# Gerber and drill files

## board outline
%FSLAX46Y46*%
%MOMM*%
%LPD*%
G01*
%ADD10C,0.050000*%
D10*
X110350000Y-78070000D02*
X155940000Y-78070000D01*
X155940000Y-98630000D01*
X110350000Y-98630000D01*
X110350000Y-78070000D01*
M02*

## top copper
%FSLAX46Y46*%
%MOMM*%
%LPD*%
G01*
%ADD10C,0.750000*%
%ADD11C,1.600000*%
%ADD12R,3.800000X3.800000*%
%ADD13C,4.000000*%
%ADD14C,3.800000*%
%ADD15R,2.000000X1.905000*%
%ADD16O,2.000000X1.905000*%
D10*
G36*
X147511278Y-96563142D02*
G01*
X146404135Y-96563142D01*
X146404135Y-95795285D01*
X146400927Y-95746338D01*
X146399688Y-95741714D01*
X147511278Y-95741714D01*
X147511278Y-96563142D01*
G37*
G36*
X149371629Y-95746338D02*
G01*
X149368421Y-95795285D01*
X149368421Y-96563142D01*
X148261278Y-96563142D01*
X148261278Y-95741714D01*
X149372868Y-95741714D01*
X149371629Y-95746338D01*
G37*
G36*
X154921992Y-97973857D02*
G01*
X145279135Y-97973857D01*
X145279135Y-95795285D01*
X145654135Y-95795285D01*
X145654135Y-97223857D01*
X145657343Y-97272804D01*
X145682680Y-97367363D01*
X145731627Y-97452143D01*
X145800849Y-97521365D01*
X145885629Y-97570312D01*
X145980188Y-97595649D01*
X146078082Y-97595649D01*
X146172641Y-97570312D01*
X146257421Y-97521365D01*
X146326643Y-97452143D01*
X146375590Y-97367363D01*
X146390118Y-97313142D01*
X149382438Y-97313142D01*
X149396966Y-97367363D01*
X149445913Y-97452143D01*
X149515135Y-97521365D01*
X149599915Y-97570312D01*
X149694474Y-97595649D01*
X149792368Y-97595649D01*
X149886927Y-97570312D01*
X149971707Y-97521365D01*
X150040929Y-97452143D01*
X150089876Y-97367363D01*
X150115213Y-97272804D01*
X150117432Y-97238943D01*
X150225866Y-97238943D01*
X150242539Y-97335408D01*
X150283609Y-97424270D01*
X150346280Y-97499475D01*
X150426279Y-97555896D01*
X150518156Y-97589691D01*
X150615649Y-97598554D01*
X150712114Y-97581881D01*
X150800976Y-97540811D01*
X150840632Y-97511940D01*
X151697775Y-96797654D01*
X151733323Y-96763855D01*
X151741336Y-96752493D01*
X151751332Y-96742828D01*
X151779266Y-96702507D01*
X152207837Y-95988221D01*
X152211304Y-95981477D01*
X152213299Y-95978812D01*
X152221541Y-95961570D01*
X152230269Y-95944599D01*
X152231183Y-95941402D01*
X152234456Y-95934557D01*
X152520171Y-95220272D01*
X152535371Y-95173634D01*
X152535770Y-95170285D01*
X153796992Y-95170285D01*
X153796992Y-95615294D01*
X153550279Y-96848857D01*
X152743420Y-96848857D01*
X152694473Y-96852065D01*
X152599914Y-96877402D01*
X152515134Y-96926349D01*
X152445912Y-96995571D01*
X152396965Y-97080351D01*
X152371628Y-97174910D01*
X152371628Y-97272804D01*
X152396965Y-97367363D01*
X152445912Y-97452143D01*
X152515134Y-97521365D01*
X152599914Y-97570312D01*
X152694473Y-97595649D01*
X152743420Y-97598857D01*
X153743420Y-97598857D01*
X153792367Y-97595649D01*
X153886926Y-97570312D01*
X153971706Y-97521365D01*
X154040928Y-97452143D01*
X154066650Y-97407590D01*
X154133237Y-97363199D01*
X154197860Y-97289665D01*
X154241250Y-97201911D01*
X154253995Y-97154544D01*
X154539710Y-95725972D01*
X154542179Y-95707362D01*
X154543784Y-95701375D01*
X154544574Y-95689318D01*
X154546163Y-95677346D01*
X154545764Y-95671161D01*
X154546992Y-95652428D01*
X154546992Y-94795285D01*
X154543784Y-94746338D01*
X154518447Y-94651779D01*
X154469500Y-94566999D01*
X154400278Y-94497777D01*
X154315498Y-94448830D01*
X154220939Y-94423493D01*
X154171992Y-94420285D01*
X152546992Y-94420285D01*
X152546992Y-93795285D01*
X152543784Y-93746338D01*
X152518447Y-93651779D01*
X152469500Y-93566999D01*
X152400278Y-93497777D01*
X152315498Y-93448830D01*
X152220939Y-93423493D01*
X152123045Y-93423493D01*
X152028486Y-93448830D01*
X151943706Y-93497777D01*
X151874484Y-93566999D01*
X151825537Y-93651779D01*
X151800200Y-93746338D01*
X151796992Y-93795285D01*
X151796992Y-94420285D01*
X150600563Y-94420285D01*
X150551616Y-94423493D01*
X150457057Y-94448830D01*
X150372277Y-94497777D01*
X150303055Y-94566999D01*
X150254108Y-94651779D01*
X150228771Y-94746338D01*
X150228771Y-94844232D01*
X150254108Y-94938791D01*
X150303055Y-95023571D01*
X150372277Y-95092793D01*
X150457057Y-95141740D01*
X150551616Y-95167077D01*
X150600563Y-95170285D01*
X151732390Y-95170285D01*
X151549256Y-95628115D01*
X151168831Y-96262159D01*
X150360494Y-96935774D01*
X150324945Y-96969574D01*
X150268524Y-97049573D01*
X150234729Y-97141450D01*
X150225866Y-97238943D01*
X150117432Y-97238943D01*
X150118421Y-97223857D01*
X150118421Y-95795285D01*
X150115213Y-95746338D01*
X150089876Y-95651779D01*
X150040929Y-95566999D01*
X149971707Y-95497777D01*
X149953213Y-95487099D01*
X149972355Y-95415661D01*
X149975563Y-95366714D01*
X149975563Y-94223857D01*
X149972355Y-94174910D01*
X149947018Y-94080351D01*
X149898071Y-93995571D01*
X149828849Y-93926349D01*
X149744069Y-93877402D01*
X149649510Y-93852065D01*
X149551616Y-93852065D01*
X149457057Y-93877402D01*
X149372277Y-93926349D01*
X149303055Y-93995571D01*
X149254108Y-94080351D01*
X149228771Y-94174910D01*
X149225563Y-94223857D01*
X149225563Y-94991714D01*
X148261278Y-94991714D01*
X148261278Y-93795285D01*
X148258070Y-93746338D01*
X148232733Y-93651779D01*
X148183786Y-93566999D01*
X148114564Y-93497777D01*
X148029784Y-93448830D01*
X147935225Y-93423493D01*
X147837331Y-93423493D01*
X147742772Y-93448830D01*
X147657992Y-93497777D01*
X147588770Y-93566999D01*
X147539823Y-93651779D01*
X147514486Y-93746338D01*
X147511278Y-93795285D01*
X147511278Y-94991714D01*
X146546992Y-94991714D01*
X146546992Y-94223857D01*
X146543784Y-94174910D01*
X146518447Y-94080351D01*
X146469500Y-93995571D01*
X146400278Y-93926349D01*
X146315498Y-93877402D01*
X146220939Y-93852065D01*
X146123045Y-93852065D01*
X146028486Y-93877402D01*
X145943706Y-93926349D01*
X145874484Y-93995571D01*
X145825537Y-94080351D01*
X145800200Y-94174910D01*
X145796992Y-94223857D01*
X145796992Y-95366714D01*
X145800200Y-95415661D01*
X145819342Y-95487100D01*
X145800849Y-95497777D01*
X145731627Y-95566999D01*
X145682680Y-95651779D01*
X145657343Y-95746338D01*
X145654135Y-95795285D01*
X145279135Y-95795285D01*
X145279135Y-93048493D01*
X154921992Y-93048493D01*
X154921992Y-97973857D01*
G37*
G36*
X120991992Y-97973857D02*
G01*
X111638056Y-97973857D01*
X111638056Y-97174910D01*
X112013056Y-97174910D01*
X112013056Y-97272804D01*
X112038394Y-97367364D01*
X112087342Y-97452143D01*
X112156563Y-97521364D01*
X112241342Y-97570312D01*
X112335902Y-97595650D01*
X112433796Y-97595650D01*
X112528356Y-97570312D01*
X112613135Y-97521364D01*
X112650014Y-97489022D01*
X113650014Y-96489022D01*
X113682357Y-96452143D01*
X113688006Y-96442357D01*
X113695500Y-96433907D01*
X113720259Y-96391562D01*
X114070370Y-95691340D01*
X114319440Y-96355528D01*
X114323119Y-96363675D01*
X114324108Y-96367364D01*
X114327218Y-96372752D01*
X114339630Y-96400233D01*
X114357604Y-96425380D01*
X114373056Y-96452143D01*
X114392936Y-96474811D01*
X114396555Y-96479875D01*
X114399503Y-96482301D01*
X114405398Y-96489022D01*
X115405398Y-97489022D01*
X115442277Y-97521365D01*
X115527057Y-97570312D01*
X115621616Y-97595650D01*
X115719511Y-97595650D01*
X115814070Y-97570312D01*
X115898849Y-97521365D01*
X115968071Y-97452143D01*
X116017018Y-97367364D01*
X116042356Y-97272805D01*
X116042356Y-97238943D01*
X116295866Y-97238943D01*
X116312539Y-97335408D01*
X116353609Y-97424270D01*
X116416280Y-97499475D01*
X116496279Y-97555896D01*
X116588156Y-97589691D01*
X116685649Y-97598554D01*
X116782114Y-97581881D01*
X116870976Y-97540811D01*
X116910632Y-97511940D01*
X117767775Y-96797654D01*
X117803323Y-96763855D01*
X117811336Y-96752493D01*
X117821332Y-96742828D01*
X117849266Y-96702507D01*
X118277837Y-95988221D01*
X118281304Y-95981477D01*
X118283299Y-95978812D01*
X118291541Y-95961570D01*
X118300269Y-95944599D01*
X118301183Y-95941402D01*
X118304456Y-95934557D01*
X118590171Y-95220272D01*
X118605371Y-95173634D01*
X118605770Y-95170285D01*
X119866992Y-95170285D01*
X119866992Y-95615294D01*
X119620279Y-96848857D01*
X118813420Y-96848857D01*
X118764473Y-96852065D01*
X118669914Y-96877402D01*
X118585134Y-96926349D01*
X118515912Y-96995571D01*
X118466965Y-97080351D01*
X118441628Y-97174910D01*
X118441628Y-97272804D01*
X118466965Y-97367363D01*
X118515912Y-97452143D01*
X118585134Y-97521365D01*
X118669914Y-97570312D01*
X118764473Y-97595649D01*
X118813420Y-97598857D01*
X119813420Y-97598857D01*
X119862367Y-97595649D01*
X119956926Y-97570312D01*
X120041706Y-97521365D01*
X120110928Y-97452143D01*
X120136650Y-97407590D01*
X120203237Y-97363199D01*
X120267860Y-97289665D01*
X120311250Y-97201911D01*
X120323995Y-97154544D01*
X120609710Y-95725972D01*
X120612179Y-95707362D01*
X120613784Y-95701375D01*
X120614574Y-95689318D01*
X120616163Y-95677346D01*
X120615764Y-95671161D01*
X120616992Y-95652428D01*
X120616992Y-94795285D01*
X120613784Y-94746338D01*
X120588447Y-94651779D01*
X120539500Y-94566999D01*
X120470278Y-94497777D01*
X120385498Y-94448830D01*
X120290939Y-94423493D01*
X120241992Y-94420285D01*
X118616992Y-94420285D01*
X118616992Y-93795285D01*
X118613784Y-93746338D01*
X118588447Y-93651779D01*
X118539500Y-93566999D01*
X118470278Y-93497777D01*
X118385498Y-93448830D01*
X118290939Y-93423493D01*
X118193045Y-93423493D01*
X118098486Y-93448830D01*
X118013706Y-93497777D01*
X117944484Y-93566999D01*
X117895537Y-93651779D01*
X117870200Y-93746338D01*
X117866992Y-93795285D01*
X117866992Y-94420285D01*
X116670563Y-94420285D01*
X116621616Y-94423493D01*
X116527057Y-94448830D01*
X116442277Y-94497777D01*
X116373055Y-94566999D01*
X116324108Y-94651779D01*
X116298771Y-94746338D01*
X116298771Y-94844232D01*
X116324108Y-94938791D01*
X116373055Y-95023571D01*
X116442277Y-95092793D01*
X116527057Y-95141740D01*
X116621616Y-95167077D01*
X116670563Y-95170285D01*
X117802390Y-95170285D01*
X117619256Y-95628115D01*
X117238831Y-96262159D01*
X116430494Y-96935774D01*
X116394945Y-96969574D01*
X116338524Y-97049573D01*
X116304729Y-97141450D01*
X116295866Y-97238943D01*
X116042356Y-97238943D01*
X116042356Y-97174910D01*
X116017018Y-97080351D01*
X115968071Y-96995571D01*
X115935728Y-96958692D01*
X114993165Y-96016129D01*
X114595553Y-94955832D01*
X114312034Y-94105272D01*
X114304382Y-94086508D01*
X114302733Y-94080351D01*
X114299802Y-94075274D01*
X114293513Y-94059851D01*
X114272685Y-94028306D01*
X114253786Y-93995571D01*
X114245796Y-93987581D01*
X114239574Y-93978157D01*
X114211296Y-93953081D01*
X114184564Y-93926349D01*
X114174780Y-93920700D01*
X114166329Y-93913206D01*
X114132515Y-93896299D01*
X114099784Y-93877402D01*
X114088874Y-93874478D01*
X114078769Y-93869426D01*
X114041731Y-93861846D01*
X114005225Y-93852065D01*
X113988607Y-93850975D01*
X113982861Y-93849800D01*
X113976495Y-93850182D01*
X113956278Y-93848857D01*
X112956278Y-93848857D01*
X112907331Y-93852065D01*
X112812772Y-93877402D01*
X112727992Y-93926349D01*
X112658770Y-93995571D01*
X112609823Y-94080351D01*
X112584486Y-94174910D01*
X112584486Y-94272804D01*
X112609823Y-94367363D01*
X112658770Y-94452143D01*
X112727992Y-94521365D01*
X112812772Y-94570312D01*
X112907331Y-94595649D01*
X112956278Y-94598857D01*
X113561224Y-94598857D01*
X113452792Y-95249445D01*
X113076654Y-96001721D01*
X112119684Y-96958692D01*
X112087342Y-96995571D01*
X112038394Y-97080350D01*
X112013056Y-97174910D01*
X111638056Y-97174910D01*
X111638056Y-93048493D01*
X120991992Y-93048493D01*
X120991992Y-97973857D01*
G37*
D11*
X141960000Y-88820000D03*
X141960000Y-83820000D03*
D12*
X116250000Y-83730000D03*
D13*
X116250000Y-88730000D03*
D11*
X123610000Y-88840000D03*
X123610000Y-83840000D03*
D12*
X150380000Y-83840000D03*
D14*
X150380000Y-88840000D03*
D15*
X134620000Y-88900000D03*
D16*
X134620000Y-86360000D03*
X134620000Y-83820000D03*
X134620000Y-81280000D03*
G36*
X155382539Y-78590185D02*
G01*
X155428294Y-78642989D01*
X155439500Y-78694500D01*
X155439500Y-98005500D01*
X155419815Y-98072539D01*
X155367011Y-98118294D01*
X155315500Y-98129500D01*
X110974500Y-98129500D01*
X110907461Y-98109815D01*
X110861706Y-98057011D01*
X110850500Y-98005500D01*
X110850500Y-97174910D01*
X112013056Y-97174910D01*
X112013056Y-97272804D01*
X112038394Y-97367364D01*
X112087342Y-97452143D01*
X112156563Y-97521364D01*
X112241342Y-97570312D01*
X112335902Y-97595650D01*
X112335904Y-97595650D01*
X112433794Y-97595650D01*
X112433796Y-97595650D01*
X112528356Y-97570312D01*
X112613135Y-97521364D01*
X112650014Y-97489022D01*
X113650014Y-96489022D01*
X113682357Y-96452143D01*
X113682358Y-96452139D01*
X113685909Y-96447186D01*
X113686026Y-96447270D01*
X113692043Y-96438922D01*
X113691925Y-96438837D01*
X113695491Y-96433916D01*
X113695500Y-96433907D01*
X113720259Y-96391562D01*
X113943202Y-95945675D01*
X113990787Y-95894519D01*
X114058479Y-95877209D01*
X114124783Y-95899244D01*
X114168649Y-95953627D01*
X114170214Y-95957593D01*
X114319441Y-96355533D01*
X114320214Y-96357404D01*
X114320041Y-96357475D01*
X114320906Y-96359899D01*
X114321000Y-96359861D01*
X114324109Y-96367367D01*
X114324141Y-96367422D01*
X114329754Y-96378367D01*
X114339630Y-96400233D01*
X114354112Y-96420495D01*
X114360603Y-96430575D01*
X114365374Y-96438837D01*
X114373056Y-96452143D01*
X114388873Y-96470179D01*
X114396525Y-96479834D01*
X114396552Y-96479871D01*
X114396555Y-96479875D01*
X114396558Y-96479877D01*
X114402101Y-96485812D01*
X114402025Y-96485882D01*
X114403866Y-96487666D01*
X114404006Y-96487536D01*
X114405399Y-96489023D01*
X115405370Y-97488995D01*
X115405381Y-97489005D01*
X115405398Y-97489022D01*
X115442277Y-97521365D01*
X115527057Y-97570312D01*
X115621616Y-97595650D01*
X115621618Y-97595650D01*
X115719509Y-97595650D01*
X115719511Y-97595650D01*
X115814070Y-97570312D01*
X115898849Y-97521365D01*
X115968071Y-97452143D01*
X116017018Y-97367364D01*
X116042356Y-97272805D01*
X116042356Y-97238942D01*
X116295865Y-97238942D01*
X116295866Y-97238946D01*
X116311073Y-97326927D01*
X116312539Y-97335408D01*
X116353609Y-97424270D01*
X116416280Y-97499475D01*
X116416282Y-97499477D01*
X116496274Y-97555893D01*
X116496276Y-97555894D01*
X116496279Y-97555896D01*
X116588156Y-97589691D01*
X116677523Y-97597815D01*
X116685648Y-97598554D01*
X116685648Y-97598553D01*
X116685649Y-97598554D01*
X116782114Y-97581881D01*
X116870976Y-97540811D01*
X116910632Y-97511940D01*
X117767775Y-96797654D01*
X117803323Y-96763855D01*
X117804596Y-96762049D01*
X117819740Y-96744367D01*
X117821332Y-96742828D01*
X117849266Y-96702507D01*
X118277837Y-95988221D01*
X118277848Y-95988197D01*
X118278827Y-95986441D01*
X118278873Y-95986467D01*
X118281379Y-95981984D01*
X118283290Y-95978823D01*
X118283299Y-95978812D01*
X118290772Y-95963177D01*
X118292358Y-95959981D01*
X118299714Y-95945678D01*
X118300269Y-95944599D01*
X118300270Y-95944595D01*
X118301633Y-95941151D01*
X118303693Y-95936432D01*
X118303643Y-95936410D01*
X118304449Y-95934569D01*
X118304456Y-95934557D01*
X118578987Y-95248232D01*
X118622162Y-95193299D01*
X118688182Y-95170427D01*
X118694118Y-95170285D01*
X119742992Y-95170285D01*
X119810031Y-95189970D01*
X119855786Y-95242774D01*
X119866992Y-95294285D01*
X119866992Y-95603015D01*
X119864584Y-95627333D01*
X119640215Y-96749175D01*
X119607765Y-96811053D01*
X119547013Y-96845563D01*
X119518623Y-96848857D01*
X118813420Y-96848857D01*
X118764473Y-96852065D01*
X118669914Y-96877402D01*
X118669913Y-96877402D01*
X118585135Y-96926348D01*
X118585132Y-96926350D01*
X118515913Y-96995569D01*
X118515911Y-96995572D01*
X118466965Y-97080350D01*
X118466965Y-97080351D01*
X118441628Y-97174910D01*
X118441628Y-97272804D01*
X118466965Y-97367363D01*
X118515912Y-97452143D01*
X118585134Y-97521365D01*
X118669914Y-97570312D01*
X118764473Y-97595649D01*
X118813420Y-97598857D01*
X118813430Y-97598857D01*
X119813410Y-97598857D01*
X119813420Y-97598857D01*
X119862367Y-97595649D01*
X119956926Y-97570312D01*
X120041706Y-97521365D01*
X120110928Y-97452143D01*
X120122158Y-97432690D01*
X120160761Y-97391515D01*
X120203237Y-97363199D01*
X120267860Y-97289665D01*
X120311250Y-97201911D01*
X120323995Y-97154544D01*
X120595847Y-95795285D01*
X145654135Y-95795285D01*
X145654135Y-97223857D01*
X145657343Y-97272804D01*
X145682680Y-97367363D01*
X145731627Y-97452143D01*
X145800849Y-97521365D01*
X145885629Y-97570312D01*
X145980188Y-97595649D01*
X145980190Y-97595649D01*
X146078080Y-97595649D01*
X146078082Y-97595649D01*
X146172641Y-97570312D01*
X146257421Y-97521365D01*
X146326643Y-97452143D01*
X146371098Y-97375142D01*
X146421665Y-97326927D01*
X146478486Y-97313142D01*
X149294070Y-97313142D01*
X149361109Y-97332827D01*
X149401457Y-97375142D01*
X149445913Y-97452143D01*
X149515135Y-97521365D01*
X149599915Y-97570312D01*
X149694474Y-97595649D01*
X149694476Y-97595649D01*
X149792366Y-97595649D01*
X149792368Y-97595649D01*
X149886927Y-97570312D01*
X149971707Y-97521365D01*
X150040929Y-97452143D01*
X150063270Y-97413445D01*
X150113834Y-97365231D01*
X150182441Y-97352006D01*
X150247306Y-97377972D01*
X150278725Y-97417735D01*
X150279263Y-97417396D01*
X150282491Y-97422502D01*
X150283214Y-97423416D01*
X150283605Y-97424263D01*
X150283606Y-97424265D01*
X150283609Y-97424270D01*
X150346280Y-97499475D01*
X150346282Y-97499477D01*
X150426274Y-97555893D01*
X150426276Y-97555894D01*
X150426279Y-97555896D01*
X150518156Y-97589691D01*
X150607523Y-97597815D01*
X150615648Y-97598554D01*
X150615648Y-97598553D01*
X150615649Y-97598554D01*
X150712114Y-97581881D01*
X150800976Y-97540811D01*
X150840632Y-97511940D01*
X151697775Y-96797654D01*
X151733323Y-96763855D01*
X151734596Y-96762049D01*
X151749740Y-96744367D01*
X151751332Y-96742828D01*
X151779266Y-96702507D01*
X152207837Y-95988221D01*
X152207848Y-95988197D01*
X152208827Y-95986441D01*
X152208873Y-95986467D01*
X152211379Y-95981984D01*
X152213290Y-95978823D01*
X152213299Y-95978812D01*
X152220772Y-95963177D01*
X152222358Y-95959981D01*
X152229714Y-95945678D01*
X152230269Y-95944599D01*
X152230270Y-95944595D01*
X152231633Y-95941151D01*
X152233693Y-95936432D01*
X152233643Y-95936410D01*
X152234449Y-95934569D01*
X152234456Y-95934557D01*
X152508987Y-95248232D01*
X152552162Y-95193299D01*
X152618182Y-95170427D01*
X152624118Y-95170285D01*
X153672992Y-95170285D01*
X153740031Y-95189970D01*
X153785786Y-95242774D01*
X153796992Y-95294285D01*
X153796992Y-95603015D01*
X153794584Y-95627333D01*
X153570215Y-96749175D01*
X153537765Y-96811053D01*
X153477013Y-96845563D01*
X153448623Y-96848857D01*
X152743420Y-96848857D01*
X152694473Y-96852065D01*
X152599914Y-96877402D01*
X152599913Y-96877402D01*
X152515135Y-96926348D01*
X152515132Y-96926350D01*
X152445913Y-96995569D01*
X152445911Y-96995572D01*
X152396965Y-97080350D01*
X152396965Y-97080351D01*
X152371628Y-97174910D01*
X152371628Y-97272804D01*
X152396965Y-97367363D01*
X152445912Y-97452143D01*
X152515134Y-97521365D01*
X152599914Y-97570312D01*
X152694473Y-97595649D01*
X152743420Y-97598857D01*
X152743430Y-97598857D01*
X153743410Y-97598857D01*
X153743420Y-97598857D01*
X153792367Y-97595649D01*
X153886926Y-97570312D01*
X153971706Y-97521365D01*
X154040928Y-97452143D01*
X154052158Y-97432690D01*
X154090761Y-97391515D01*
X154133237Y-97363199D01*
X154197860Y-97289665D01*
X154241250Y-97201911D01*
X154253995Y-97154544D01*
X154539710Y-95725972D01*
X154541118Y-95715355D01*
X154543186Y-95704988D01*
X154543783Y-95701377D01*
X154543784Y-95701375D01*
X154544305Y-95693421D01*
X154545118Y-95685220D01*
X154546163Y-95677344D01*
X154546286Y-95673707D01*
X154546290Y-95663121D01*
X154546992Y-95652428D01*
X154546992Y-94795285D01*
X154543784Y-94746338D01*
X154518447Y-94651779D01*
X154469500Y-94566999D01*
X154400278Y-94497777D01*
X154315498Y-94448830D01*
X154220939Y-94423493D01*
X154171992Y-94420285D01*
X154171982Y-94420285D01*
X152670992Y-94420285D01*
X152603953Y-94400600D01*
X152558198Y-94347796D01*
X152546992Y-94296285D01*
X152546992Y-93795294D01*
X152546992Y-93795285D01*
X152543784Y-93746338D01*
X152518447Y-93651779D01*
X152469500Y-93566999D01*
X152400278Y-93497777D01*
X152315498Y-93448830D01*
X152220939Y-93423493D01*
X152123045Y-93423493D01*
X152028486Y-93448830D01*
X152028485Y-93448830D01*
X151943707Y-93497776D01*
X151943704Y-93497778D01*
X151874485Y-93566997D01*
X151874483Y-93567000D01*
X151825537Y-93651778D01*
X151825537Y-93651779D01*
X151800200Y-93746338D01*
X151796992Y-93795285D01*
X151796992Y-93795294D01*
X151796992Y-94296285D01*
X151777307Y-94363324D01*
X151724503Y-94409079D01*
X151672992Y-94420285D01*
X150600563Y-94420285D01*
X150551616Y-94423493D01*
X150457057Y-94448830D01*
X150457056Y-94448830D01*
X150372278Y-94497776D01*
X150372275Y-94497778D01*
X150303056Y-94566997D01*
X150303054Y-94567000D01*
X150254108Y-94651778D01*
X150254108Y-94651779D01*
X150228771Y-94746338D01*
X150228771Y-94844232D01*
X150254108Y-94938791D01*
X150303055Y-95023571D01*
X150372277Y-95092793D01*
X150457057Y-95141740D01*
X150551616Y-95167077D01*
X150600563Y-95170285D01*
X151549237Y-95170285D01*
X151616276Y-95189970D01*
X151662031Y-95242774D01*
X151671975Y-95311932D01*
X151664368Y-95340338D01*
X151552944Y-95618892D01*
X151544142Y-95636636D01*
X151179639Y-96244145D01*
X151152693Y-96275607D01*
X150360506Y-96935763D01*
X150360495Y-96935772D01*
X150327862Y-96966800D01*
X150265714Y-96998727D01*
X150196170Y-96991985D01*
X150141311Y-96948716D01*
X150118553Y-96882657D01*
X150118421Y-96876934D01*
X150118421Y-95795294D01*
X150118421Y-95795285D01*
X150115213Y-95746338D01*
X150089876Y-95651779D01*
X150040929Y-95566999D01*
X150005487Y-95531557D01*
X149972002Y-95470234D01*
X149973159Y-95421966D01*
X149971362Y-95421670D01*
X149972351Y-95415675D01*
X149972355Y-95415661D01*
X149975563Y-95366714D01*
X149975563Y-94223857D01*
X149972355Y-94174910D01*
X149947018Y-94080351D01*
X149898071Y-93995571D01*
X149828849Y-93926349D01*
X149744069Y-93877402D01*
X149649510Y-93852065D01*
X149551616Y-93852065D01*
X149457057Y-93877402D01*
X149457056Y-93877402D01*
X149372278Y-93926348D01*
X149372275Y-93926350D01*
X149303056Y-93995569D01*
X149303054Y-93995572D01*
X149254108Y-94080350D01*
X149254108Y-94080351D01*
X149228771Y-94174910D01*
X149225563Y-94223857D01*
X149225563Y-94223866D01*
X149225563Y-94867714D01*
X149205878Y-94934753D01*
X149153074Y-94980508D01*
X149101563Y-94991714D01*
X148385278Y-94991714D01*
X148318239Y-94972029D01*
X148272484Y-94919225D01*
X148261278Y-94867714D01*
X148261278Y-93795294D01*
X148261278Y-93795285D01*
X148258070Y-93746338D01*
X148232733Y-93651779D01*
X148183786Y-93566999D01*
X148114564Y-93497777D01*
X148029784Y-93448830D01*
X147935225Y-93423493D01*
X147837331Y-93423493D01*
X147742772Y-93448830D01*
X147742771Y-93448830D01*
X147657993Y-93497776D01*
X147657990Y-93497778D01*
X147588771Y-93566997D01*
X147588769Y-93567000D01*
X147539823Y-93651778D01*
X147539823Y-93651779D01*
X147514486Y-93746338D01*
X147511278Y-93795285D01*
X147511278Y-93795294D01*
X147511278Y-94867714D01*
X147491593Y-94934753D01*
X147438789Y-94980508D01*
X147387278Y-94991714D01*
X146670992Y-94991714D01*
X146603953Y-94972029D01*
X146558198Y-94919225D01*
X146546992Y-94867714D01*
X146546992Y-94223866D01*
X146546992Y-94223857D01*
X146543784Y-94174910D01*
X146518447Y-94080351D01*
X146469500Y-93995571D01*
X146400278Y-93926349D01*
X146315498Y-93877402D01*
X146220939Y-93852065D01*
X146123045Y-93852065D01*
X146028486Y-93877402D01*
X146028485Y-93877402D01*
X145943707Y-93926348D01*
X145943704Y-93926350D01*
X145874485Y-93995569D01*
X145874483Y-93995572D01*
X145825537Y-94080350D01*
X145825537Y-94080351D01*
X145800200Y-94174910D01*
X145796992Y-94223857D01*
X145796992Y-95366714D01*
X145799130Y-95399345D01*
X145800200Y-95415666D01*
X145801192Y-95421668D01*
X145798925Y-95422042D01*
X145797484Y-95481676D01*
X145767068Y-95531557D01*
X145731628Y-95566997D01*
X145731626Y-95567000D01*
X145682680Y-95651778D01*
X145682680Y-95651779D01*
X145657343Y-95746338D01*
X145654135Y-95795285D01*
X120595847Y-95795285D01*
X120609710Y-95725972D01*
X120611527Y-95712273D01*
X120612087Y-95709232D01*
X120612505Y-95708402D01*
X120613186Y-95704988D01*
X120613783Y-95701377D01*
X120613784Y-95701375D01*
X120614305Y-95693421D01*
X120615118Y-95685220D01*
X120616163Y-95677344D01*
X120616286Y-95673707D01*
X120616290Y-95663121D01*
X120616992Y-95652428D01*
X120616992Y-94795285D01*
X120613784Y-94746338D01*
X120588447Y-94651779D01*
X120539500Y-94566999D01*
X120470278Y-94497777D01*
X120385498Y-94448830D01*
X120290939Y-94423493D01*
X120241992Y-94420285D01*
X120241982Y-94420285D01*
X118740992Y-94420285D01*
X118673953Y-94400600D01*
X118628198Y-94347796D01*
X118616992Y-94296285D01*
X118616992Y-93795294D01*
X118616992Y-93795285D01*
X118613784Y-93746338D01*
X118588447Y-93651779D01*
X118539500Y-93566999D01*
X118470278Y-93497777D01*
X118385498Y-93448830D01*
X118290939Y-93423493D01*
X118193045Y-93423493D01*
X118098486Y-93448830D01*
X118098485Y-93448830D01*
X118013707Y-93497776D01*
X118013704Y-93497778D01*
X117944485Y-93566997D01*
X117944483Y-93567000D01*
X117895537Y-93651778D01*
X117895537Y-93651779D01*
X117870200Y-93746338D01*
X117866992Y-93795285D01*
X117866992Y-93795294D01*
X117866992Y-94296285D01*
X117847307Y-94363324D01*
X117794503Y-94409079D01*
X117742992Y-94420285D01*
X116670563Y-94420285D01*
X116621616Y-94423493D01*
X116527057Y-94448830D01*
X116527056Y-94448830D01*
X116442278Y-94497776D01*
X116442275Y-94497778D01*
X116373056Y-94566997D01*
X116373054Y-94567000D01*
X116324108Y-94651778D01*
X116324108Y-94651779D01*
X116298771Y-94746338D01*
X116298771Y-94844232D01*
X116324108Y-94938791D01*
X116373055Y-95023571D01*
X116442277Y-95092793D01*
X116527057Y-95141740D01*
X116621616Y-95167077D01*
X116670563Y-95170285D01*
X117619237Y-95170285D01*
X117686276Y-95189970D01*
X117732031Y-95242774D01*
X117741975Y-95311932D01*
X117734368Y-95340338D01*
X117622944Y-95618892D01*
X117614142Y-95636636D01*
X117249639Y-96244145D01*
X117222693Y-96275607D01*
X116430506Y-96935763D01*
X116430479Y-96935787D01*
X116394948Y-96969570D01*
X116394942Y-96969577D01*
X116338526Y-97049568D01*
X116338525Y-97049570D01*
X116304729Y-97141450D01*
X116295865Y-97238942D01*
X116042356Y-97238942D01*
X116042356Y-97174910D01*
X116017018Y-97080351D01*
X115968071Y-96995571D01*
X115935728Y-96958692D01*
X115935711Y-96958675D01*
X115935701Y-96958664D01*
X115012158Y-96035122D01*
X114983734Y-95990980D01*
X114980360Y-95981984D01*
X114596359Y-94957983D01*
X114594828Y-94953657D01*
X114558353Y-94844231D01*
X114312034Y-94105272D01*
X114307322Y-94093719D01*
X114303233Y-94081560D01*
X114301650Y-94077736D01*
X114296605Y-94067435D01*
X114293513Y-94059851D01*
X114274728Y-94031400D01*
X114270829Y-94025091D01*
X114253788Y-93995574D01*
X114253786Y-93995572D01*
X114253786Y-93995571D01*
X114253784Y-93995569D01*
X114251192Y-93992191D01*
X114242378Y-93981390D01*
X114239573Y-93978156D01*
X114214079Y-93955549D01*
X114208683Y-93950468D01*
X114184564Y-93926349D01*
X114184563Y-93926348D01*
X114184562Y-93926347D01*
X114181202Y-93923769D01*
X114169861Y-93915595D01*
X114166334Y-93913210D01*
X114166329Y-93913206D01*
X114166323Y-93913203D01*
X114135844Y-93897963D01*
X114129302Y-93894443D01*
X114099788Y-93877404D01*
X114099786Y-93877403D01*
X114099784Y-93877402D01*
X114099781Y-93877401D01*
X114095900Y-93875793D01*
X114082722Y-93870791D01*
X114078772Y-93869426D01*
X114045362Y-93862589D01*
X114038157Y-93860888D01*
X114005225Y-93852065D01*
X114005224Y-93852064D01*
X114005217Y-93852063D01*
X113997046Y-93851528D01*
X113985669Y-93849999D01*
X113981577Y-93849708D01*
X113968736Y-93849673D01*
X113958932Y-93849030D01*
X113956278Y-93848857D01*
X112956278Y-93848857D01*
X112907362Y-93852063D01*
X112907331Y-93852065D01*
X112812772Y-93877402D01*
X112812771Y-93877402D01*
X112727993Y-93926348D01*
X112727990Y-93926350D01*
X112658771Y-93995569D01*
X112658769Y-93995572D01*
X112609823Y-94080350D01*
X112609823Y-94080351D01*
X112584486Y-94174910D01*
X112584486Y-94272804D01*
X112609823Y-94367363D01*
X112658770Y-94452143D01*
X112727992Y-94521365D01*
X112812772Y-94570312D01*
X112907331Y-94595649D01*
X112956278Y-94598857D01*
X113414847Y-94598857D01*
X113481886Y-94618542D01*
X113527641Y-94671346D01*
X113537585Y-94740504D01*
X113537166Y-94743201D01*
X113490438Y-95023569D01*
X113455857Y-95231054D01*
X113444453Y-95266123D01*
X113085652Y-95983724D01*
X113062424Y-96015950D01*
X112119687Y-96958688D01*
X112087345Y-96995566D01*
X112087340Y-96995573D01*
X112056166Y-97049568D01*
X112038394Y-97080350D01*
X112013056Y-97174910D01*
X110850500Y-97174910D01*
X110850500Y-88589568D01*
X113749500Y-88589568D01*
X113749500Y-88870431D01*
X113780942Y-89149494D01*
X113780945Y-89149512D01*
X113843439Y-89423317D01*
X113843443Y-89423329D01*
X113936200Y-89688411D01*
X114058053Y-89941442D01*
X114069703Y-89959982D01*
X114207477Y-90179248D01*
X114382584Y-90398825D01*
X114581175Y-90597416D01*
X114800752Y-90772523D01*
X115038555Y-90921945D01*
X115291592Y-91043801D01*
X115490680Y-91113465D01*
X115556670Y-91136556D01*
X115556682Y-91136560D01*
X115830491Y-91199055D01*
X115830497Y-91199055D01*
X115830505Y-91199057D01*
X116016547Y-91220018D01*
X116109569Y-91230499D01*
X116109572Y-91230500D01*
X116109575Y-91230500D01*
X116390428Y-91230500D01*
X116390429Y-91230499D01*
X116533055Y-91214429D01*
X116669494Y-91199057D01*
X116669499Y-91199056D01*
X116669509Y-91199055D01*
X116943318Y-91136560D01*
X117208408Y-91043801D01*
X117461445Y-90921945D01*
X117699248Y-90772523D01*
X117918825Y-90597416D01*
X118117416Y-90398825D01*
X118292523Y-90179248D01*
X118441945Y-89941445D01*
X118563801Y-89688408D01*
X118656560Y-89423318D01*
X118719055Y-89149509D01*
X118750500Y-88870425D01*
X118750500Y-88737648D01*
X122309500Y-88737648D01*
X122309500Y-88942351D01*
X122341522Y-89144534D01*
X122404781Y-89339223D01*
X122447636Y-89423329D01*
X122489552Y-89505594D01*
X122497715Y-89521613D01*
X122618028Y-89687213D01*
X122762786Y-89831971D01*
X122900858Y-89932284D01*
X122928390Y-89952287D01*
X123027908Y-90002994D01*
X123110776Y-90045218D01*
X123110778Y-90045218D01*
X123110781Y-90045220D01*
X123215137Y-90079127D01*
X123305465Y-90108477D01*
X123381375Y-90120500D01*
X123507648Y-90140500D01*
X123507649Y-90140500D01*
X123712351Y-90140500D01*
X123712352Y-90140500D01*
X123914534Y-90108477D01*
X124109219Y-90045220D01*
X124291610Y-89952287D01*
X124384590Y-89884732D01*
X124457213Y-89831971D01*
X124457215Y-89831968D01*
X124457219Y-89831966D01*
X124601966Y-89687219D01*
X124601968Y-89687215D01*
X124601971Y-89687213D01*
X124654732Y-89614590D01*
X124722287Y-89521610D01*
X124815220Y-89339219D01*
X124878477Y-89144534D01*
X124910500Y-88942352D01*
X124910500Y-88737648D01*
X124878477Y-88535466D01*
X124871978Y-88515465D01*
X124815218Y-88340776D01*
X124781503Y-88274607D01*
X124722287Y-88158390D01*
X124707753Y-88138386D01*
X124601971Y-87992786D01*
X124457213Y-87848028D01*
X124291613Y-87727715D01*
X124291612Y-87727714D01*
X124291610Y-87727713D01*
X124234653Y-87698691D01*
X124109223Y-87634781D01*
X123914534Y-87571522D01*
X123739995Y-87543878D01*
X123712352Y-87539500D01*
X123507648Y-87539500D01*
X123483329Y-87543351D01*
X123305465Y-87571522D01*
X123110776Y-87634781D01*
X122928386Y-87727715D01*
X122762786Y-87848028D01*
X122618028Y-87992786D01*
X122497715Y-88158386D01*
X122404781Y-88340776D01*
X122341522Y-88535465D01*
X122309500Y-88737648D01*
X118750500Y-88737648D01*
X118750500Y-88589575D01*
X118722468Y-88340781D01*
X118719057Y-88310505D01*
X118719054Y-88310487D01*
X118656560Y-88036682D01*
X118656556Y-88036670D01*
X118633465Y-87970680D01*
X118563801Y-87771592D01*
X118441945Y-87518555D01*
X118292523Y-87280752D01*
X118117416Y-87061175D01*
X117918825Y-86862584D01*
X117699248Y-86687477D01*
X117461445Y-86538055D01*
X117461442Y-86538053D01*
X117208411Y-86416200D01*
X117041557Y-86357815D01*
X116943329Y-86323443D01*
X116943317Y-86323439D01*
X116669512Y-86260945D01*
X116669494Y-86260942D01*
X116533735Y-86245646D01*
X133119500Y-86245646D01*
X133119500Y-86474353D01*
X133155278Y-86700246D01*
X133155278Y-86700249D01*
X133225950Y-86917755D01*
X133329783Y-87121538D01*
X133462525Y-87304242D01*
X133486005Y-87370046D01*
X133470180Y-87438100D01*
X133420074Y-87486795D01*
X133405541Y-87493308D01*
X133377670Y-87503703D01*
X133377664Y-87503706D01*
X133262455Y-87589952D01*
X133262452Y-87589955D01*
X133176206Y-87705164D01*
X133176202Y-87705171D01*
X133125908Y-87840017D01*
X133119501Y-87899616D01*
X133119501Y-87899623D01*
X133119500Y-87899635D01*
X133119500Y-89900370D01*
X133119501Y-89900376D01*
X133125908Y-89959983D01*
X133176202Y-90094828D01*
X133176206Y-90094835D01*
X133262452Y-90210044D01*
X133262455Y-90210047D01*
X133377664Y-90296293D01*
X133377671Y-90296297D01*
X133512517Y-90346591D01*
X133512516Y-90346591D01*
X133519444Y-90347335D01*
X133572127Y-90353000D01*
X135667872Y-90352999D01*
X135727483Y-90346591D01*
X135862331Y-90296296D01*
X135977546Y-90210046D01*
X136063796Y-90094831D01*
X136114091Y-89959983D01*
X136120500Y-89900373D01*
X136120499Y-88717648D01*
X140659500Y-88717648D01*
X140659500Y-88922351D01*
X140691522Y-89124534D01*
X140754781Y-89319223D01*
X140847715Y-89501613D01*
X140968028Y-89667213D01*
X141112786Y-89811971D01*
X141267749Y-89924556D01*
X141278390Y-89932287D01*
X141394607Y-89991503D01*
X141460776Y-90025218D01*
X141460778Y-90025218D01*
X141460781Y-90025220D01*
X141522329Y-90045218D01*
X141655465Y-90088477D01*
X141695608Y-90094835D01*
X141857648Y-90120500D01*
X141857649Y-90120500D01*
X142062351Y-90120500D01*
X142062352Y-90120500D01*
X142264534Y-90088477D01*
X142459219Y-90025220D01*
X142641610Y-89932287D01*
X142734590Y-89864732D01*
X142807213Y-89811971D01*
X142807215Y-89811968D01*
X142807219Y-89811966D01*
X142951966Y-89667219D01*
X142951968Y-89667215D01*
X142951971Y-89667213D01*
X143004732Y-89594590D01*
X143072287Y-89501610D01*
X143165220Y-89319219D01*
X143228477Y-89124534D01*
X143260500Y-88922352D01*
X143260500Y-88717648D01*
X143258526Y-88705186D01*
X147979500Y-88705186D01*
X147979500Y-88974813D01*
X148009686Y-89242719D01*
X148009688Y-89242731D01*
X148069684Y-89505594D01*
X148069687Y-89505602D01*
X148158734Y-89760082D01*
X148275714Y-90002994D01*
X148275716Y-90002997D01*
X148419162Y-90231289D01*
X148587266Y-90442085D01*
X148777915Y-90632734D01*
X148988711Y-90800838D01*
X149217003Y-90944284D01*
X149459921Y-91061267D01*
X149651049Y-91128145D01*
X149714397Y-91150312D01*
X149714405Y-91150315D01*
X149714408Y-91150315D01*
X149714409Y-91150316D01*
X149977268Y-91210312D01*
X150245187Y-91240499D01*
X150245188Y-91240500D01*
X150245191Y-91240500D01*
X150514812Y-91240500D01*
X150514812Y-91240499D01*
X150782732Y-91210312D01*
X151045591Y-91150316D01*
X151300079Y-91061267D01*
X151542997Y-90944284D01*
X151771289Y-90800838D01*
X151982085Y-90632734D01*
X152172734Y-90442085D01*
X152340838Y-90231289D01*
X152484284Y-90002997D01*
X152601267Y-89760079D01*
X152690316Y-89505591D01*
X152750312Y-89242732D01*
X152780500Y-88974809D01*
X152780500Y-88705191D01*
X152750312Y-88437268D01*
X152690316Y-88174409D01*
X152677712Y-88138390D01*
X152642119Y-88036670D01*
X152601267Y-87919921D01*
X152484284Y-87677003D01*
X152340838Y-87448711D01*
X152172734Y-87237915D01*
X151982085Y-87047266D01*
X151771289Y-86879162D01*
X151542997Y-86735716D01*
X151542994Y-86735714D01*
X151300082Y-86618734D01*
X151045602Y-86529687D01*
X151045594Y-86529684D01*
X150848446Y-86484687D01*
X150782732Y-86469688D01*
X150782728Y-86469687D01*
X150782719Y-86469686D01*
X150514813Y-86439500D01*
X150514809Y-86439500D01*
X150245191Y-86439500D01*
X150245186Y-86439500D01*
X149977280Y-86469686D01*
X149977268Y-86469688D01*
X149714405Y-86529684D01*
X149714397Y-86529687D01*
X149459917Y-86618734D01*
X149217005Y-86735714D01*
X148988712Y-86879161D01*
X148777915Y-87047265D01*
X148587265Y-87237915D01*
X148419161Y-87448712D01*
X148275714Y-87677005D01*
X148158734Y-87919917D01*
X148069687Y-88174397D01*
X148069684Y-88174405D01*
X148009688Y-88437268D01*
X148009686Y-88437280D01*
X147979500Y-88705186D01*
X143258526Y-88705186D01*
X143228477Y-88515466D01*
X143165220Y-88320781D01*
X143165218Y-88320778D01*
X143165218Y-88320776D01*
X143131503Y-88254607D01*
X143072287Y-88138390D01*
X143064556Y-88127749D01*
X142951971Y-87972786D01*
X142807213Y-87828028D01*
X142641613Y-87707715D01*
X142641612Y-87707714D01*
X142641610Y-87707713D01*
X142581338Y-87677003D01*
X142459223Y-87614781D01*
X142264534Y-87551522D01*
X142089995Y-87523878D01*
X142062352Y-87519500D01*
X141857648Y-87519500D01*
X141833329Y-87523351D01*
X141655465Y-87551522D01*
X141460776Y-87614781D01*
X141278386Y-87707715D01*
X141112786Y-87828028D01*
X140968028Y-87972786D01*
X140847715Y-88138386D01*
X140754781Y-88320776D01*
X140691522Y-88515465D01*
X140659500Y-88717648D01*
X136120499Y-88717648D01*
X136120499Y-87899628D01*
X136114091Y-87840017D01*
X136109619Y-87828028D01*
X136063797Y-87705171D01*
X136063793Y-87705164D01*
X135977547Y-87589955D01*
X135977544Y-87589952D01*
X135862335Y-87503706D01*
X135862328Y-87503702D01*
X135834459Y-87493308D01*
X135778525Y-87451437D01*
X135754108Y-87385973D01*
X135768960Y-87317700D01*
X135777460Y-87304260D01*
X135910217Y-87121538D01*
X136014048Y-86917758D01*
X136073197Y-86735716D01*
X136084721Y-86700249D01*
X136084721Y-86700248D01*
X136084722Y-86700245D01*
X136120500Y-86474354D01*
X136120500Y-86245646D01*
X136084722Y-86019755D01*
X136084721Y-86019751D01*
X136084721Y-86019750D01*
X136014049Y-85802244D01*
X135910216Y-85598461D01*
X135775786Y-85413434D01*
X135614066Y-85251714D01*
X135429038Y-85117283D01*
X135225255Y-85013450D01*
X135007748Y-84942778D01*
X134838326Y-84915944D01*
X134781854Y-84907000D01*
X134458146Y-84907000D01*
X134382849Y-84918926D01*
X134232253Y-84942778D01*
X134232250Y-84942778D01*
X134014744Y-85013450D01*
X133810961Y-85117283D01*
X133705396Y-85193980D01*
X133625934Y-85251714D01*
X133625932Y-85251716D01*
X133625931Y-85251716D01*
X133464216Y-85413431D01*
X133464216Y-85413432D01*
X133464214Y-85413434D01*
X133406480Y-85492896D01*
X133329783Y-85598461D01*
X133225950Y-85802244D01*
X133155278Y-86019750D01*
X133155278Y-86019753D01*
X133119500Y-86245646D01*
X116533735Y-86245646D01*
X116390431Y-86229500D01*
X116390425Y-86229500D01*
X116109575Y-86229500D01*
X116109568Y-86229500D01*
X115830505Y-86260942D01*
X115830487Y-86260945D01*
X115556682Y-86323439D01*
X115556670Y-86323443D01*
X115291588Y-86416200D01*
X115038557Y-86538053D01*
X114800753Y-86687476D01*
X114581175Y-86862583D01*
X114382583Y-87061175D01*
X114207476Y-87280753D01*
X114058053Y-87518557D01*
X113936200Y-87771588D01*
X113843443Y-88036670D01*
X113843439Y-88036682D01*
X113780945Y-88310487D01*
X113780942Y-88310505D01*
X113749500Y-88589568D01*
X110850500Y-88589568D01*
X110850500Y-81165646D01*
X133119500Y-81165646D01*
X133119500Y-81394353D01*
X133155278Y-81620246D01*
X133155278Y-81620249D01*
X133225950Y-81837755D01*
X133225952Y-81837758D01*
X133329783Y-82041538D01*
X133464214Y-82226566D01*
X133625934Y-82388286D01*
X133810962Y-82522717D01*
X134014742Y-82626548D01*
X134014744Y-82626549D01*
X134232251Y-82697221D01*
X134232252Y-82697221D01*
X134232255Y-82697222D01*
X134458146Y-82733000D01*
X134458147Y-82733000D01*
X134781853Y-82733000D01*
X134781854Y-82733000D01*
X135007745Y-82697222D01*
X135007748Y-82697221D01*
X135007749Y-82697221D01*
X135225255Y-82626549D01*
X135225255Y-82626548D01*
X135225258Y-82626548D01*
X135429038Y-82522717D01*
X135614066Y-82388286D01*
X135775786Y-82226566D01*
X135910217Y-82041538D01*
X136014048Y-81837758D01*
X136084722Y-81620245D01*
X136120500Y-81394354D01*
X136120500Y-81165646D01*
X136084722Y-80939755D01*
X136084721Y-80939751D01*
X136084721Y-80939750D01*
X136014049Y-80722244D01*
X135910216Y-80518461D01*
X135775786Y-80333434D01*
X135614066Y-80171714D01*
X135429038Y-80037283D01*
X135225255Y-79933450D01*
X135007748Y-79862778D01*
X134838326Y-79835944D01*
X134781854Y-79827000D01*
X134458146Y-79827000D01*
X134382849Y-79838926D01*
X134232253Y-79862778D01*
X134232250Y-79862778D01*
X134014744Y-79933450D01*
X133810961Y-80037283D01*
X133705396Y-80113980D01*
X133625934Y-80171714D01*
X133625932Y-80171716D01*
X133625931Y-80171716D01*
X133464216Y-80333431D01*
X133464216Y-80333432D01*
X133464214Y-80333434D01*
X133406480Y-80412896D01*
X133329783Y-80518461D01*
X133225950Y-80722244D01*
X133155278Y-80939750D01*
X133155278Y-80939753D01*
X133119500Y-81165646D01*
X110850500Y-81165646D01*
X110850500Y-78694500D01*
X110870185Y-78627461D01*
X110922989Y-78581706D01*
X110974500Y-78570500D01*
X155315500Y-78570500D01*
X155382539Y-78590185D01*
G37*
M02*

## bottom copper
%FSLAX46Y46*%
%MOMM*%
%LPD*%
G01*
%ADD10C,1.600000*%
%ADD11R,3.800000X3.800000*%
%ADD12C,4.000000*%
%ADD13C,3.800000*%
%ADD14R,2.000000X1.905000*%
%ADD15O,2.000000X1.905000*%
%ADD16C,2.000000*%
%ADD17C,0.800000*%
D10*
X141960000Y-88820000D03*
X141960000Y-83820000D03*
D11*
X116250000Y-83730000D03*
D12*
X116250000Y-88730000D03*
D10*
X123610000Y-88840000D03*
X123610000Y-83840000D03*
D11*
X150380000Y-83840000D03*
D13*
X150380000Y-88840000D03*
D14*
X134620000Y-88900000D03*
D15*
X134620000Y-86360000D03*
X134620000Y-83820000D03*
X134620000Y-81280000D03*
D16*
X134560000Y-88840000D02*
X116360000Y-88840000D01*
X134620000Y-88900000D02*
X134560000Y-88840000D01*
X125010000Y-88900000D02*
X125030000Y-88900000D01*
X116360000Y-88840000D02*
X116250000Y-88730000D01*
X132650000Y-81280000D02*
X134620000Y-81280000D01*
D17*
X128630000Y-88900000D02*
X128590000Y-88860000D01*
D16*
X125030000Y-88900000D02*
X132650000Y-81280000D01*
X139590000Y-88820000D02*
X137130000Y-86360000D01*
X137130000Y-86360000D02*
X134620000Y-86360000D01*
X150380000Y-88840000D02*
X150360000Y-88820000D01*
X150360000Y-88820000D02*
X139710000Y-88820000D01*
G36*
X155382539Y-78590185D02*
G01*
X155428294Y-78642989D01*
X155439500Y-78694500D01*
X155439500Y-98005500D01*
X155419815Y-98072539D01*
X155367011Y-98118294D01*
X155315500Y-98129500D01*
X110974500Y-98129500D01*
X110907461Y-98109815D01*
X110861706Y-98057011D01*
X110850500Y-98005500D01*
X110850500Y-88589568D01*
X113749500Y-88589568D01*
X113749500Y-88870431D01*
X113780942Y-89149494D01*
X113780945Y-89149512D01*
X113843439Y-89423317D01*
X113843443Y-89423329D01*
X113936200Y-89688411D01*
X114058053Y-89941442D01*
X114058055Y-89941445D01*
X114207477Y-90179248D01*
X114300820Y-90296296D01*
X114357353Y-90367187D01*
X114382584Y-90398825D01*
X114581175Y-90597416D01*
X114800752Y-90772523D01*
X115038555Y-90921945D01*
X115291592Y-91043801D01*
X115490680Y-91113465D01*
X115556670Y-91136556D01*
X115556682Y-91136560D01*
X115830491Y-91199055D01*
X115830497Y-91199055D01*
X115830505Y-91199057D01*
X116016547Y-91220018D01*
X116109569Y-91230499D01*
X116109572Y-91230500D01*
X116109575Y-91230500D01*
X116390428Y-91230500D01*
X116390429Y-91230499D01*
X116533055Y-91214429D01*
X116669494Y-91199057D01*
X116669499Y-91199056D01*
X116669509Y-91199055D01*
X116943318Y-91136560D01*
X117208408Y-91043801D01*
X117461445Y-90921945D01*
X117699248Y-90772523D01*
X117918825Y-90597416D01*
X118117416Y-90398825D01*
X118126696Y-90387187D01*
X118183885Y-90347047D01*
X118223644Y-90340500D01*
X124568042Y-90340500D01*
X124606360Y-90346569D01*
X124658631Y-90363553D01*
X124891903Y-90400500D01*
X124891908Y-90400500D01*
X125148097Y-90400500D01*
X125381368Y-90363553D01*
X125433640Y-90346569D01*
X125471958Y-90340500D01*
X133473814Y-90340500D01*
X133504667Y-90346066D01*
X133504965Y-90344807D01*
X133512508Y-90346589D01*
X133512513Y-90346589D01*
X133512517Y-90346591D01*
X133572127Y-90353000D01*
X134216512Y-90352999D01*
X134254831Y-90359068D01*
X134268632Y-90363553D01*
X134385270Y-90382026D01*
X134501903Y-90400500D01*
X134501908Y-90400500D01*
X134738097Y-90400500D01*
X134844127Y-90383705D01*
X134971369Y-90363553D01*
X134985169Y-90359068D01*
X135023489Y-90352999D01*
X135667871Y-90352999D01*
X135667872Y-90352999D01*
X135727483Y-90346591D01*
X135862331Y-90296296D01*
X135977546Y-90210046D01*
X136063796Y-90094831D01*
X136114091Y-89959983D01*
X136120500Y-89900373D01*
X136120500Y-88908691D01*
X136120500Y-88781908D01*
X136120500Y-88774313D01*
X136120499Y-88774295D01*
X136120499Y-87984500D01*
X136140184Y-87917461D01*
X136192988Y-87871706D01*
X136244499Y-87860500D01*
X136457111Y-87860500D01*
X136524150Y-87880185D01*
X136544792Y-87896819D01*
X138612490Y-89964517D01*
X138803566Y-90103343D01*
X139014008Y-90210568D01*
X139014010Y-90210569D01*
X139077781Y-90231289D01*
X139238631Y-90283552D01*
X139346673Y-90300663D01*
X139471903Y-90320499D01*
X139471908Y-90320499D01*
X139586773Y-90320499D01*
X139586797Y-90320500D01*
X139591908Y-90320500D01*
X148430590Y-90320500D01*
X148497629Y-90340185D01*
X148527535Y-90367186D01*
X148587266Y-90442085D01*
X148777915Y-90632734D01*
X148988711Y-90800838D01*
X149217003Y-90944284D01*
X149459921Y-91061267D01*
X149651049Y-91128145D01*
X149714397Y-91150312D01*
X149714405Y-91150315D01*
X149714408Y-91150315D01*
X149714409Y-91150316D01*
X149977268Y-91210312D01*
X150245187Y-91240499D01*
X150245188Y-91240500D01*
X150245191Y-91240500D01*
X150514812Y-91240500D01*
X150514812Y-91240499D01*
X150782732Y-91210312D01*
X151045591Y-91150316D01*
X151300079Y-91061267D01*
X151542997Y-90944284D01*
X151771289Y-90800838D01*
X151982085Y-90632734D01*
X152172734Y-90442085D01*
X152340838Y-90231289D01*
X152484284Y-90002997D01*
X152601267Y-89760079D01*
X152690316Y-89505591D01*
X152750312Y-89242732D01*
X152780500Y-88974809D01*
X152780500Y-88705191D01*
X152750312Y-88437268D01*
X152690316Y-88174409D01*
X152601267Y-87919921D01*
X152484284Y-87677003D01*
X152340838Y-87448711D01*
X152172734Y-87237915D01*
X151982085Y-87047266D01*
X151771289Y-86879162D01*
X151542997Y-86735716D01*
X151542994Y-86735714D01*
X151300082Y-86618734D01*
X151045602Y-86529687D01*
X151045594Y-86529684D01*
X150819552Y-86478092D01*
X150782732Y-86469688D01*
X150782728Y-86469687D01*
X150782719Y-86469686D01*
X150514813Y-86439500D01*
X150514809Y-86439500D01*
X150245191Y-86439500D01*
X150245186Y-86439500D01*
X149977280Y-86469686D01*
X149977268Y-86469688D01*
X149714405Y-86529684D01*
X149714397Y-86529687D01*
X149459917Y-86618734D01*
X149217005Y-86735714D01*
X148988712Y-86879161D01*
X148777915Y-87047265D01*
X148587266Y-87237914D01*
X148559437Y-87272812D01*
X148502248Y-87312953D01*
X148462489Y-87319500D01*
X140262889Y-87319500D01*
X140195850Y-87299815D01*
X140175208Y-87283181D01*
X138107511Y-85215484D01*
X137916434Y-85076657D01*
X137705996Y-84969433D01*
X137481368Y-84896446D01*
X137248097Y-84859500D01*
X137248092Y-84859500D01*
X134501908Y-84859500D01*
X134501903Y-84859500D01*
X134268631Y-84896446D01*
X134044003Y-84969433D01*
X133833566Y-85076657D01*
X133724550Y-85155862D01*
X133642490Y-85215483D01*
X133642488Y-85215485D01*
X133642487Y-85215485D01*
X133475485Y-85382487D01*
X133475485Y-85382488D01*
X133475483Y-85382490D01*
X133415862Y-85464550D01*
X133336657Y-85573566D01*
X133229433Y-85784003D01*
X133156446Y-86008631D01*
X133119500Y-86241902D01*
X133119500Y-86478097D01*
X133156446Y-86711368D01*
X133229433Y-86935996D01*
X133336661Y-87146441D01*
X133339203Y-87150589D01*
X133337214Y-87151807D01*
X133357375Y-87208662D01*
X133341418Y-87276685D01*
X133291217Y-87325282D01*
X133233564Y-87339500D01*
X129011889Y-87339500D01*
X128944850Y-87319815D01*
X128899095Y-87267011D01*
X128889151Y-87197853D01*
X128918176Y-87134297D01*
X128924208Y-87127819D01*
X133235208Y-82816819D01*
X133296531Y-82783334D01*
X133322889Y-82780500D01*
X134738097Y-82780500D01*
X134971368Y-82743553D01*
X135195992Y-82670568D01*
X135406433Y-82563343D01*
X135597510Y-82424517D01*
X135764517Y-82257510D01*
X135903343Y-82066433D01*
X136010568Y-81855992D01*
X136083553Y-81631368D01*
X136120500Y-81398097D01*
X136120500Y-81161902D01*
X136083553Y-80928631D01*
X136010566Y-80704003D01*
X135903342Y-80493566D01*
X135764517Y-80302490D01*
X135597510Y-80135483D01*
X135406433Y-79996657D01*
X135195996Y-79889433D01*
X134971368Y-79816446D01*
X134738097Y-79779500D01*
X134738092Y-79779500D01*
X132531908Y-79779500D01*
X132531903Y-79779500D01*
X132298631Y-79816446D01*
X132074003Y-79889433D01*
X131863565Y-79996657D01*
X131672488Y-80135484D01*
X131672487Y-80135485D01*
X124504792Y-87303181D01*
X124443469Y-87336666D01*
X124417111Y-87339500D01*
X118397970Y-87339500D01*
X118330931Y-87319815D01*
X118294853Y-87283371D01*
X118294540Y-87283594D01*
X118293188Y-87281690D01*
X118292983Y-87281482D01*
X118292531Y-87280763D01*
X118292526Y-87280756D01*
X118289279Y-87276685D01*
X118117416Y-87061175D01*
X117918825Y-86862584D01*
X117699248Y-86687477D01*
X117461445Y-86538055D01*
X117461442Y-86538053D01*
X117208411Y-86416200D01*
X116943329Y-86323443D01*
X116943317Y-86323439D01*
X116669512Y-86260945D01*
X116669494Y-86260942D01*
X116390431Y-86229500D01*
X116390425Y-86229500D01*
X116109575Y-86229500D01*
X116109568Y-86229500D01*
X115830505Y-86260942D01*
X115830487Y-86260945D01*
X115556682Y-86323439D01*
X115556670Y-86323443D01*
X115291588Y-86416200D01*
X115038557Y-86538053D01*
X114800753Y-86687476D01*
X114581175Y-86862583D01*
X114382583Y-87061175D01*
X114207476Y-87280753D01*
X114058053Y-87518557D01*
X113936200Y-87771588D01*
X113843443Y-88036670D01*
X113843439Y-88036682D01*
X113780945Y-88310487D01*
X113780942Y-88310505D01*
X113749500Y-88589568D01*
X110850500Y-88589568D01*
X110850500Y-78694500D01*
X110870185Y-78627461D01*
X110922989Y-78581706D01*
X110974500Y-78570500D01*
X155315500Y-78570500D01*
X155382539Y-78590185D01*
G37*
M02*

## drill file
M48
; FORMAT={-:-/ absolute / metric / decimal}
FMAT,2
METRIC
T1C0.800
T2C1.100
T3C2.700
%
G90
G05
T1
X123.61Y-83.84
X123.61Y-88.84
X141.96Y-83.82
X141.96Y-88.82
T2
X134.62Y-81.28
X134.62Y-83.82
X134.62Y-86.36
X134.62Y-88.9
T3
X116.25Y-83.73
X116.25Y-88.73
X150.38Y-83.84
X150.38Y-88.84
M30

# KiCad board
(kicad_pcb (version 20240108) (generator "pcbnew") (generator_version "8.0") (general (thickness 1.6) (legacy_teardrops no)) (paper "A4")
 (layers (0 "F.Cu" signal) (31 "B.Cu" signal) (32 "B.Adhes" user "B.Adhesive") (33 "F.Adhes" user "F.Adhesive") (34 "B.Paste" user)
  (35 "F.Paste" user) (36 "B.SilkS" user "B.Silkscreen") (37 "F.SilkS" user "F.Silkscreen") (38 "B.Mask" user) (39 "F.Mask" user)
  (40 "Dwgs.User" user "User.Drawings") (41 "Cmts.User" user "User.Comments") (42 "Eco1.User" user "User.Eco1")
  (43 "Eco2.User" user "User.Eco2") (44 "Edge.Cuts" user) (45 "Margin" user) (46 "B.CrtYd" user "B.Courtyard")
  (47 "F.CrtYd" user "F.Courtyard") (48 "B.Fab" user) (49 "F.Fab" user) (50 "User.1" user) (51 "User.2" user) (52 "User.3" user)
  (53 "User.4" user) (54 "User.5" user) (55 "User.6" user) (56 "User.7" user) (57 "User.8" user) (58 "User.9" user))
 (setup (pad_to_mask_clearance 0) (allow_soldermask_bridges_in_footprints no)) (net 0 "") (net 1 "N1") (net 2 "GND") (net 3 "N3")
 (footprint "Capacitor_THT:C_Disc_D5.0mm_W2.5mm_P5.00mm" (layer "F.Cu") (at 141.96 88.82 90)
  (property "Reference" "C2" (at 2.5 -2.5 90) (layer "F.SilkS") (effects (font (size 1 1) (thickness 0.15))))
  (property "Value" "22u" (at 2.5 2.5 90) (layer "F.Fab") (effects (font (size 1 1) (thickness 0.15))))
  (pad "1" thru_hole circle (at 0 0 90) (size 1.6 1.6) (drill 0.8) (layers "*.Cu" "*.Mask") (remove_unused_layers no) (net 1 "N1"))
  (pad "2" thru_hole circle (at 5 0 90) (size 1.6 1.6) (drill 0.8) (layers "*.Cu" "*.Mask") (remove_unused_layers no) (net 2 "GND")))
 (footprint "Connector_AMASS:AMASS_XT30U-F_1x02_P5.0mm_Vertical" (layer "F.Cu") (at 116.25 83.73 -90)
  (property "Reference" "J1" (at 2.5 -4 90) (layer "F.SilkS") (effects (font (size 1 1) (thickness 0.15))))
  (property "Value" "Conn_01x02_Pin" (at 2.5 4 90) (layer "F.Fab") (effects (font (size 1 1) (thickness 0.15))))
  (pad "1" thru_hole rect (at 0 0 270) (size 3.8 3.8) (drill 2.7) (layers "*.Cu" "*.Mask") (remove_unused_layers no) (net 2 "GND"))
  (pad "2" thru_hole circle (at 5 0 270) (size 4 4) (drill 2.7) (layers "*.Cu" "*.Mask") (remove_unused_layers no) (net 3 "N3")))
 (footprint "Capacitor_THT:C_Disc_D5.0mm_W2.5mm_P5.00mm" (layer "F.Cu") (at 123.61 88.84 90)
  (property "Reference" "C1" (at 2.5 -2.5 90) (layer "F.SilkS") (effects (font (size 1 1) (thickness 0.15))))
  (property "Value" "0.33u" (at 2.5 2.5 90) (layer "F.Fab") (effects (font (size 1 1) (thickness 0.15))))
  (pad "1" thru_hole circle (at 0 0 90) (size 1.6 1.6) (drill 0.8) (layers "*.Cu" "*.Mask") (remove_unused_layers no) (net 3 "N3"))
  (pad "2" thru_hole circle (at 5 0 90) (size 1.6 1.6) (drill 0.8) (layers "*.Cu" "*.Mask") (remove_unused_layers no) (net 2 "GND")))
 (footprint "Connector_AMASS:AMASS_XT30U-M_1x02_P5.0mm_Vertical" (layer "F.Cu") (at 150.38 83.84 -90)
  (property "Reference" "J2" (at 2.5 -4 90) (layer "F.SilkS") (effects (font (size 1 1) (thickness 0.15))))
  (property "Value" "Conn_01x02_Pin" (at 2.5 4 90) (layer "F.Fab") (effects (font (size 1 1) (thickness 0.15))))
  (pad "1" thru_hole rect (at 0 0 270) (size 3.8 3.8) (drill 2.7) (layers "*.Cu" "*.Mask") (remove_unused_layers no) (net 2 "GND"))
  (pad "2" thru_hole circle (at 5 0 270) (size 3.8 3.8) (drill 2.7) (layers "*.Cu" "*.Mask") (remove_unused_layers no) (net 1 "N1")))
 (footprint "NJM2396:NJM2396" (layer "F.Cu") (at 128.27 85.09 90)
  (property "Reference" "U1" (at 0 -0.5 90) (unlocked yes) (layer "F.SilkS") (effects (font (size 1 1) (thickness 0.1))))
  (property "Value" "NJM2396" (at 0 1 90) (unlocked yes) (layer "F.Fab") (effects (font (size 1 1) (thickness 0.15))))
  (pad "1" thru_hole rect (at -3.81 6.35 90) (size 1.905 2) (drill 1.1) (layers "*.Cu" "*.Mask") (remove_unused_layers no) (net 3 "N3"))
  (pad "2" thru_hole oval (at -1.27 6.35 270) (size 1.905 2) (drill 1.1) (layers "*.Cu" "*.Mask") (remove_unused_layers no) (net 1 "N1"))
  (pad "3" thru_hole oval (at 1.27 6.35 270) (size 1.905 2) (drill 1.1) (layers "*.Cu" "*.Mask") (remove_unused_layers no) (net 2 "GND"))
  (pad "4" thru_hole oval (at 3.81 6.35 270) (size 1.905 2) (drill 1.1) (layers "*.Cu" "*.Mask") (remove_unused_layers no) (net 3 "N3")))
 (gr_rect (start 110.35 78.07) (end 155.94 98.63) (stroke (width 0.05) (type default)) (fill none) (layer "Edge.Cuts"))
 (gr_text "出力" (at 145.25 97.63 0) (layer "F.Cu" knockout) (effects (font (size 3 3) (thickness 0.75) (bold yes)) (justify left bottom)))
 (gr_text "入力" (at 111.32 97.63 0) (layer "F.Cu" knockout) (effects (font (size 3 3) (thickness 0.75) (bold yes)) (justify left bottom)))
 (segment (start 134.56 88.84) (end 116.36 88.84) (width 2) (layer "B.Cu") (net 3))
 (segment (start 134.62 88.9) (end 134.56 88.84) (width 2) (layer "B.Cu") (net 3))
 (segment (start 125.01 88.9) (end 125.03 88.9) (width 2) (layer "B.Cu") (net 3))
 (segment (start 116.36 88.84) (end 116.25 88.73) (width 2) (layer "B.Cu") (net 3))
 (segment (start 132.65 81.28) (end 134.62 81.28) (width 2) (layer "B.Cu") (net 3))
 (segment (start 128.63 88.9) (end 128.59 88.86) (width 0.8) (layer "B.Cu") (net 3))
 (segment (start 125.03 88.9) (end 132.65 81.28) (width 2) (layer "B.Cu") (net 3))
 (segment (start 139.59 88.82) (end 137.13 86.36) (width 2) (layer "B.Cu") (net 1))
 (segment (start 137.13 86.36) (end 134.62 86.36) (width 2) (layer "B.Cu") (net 1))
 (segment (start 150.38 88.84) (end 150.36 88.82) (width 2) (layer "B.Cu") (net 1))
 (segment (start 150.36 88.82) (end 139.71 88.82) (width 2) (layer "B.Cu") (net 1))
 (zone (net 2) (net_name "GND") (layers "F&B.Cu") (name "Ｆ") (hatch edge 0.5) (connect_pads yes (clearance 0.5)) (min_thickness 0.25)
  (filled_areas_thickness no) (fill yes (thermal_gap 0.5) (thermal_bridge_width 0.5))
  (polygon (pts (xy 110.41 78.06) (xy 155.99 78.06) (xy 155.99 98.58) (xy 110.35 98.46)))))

